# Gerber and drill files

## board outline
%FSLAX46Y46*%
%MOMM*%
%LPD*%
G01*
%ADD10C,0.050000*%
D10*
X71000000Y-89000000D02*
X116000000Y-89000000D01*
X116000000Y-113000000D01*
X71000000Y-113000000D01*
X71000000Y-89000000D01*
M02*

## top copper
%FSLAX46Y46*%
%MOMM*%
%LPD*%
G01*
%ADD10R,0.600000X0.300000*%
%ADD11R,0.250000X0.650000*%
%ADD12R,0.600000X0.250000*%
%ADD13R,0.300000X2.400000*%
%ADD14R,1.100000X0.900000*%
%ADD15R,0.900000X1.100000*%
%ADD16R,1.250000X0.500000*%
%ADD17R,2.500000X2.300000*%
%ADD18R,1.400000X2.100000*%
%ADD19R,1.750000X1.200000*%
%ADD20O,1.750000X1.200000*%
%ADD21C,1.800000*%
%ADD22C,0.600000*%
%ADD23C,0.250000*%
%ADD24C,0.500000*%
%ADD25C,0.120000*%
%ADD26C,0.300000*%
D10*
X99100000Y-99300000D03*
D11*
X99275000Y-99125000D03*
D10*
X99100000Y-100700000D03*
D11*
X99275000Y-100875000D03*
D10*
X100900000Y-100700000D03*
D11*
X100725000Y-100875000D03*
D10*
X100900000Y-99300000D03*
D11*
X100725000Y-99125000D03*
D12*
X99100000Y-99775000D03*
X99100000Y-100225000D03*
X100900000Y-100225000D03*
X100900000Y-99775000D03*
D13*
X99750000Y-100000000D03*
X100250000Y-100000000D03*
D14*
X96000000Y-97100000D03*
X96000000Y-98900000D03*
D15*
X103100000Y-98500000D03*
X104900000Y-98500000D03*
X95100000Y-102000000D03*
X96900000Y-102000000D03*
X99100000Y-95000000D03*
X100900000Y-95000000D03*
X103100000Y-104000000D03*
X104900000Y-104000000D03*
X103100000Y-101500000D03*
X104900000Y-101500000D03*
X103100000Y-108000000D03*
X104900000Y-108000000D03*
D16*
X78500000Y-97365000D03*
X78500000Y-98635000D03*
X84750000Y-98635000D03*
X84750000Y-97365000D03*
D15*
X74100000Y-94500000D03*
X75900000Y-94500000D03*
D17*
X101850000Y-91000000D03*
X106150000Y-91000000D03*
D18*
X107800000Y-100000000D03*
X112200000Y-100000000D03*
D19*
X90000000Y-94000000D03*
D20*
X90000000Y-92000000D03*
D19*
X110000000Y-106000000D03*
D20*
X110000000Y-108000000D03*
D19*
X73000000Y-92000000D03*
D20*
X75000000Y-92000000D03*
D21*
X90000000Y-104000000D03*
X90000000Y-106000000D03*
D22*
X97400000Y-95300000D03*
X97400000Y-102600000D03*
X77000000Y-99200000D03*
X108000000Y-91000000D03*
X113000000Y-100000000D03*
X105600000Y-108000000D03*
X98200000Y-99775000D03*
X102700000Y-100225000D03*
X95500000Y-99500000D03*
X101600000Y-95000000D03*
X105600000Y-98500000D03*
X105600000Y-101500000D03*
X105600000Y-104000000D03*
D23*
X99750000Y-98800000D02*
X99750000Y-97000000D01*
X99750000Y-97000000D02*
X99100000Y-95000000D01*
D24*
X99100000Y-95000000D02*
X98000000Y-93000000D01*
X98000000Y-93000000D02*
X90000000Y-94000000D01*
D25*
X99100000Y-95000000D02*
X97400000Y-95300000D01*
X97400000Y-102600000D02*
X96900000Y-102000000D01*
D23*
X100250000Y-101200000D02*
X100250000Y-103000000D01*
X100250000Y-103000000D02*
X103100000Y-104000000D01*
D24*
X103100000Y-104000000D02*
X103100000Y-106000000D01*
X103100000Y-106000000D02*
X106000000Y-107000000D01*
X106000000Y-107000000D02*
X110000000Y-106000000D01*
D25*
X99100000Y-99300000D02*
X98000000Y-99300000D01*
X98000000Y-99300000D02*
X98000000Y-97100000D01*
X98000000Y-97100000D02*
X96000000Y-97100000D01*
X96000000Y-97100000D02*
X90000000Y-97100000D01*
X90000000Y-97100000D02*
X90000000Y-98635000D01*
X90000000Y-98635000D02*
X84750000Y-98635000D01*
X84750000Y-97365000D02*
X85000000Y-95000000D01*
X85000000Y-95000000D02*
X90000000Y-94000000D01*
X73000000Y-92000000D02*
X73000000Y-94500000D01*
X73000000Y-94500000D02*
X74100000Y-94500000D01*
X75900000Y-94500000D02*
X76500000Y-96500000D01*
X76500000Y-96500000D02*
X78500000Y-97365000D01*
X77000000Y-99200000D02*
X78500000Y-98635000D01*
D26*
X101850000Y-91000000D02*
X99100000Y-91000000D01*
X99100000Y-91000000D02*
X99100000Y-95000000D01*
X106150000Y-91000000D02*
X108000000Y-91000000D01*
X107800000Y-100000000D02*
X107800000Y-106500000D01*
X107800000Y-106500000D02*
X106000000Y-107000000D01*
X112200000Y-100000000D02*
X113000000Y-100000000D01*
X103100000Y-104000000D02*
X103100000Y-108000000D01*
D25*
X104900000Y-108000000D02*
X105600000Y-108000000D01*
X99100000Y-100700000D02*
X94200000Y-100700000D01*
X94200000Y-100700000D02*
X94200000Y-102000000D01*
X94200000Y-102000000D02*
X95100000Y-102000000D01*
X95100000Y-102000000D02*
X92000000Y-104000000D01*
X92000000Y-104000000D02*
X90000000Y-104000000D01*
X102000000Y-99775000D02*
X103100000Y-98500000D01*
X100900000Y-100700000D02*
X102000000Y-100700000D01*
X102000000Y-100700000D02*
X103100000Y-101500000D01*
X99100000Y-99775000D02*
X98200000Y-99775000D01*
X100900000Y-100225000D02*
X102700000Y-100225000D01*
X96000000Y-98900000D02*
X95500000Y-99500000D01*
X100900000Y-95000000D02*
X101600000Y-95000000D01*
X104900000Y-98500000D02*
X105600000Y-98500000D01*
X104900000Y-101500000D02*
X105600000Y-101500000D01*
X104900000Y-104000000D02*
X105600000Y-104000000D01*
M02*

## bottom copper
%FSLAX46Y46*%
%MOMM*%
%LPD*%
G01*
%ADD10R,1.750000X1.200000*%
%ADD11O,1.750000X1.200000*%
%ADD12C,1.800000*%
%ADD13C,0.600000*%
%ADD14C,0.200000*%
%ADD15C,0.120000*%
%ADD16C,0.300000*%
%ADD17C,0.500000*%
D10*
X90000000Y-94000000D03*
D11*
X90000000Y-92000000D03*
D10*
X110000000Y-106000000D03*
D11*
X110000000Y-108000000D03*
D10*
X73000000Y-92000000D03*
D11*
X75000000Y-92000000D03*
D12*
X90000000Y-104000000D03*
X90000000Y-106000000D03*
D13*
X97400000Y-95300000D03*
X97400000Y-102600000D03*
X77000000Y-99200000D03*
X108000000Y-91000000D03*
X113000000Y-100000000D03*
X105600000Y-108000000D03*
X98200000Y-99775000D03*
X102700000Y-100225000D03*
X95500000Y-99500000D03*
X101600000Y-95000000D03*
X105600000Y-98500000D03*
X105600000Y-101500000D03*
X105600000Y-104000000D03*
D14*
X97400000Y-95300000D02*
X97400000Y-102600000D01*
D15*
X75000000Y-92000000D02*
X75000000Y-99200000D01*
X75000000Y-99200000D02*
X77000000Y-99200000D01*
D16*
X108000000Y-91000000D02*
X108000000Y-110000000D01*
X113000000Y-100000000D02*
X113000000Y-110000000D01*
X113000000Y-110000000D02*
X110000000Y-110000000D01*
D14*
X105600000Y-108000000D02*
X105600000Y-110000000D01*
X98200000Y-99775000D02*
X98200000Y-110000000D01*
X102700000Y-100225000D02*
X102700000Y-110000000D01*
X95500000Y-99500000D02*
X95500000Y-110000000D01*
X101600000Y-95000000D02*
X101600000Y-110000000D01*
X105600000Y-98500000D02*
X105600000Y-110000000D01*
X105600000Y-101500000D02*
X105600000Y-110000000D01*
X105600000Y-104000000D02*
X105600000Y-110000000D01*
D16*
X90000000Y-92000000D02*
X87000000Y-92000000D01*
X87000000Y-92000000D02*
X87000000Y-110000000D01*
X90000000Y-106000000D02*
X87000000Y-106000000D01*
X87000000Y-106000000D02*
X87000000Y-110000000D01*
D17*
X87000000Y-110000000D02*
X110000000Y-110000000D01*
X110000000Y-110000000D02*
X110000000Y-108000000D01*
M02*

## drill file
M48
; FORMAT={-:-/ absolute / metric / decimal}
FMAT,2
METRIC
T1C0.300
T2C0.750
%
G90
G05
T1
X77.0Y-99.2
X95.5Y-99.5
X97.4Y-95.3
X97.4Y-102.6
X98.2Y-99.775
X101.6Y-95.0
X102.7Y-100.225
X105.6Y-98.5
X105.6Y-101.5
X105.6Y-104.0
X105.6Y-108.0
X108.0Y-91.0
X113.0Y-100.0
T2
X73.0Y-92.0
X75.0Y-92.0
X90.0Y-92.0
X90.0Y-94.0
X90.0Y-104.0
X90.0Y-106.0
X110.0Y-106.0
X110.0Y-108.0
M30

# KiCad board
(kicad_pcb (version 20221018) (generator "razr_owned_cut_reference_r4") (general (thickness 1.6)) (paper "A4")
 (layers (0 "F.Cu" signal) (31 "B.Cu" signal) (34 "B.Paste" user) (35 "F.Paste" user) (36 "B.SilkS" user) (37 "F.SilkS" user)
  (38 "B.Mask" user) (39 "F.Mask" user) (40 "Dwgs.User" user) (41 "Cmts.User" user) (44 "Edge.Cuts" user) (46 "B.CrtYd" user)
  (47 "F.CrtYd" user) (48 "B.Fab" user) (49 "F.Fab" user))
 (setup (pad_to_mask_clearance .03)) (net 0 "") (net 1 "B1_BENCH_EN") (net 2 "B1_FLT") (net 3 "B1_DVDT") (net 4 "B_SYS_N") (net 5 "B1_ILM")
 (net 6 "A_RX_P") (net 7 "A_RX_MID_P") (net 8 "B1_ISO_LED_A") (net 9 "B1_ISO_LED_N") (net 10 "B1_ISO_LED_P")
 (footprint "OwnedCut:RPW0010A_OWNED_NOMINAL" (layer "F.Cu") (at 100 100)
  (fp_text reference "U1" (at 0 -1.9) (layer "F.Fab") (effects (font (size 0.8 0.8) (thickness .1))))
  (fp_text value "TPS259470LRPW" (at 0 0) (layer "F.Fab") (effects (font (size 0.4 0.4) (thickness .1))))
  (pad "1" smd rect (at -0.9 -0.7) (size 0.6 0.3) (layers "F.Cu" "F.Paste" "F.Mask") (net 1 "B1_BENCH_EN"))
  (pad "1" smd rect (at -0.725 -0.875) (size 0.25 0.65) (layers "F.Cu" "F.Paste" "F.Mask") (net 1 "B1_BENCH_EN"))
  (pad "4" smd rect (at -0.9 0.7) (size 0.6 0.3) (layers "F.Cu" "F.Paste" "F.Mask") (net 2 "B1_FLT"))
  (pad "4" smd rect (at -0.725 0.875) (size 0.25 0.65) (layers "F.Cu" "F.Paste" "F.Mask") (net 2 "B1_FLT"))
  (pad "7" smd rect (at 0.9 0.7) (size 0.6 0.3) (layers "F.Cu" "F.Paste" "F.Mask") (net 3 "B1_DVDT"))
  (pad "7" smd rect (at 0.725 0.875) (size 0.25 0.65) (layers "F.Cu" "F.Paste" "F.Mask") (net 3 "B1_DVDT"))
  (pad "10" smd rect (at 0.9 -0.7) (size 0.6 0.3) (layers "F.Cu" "F.Paste" "F.Mask"))
  (pad "10" smd rect (at 0.725 -0.875) (size 0.25 0.65) (layers "F.Cu" "F.Paste" "F.Mask"))
  (pad "2" smd rect (at -0.9 -0.225) (size 0.6 0.25) (layers "F.Cu" "F.Paste" "F.Mask") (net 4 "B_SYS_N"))
  (pad "3" smd rect (at -0.9 0.225) (size 0.6 0.25) (layers "F.Cu" "F.Paste" "F.Mask"))
  (pad "8" smd rect (at 0.9 0.225) (size 0.6 0.25) (layers "F.Cu" "F.Paste" "F.Mask") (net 4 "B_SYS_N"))
  (pad "9" smd rect (at 0.9 -0.225) (size 0.6 0.25) (layers "F.Cu" "F.Paste" "F.Mask") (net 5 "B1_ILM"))
  (pad "5" smd rect (at -0.25 0) (size 0.3 2.4) (layers "F.Cu" "F.Paste" "F.Mask") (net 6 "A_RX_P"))
  (pad "6" smd rect (at 0.25 0) (size 0.3 2.4) (layers "F.Cu" "F.Paste" "F.Mask") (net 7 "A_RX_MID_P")))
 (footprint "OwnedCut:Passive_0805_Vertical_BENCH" (layer "F.Cu") (at 96 98)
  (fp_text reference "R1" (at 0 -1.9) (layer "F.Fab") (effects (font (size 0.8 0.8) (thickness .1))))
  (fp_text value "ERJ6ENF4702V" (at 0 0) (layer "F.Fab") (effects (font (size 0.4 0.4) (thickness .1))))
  (pad "1" smd rect (at 0 -0.9) (size 1.1 0.9) (layers "F.Cu" "F.Paste" "F.Mask") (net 1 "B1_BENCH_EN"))
  (pad "2" smd rect (at 0 0.9) (size 1.1 0.9) (layers "F.Cu" "F.Paste" "F.Mask") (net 4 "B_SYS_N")))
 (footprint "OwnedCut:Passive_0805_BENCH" (layer "F.Cu") (at 104 98.5)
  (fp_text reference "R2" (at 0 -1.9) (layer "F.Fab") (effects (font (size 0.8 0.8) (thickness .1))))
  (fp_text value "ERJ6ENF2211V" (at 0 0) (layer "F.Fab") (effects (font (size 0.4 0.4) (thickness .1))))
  (pad "1" smd rect (at -0.9 0) (size 0.9 1.1) (layers "F.Cu" "F.Paste" "F.Mask") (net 5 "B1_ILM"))
  (pad "2" smd rect (at 0.9 0) (size 0.9 1.1) (layers "F.Cu" "F.Paste" "F.Mask") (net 4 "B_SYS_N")))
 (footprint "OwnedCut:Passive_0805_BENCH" (layer "F.Cu") (at 96 102)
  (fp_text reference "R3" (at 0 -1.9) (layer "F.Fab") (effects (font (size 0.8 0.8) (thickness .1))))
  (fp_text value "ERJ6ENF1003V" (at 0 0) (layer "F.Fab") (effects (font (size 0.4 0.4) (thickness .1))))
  (pad "1" smd rect (at -0.9 0) (size 0.9 1.1) (layers "F.Cu" "F.Paste" "F.Mask") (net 2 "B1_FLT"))
  (pad "2" smd rect (at 0.9 0) (size 0.9 1.1) (layers "F.Cu" "F.Paste" "F.Mask") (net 6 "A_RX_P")))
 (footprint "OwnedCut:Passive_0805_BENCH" (layer "F.Cu") (at 100 95)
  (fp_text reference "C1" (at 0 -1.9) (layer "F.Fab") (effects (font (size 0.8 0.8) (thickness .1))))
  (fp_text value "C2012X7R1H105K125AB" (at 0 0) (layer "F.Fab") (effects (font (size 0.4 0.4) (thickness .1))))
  (pad "1" smd rect (at -0.9 0) (size 0.9 1.1) (layers "F.Cu" "F.Paste" "F.Mask") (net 6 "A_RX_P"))
  (pad "2" smd rect (at 0.9 0) (size 0.9 1.1) (layers "F.Cu" "F.Paste" "F.Mask") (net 4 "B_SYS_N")))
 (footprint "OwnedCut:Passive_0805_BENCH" (layer "F.Cu") (at 104 104)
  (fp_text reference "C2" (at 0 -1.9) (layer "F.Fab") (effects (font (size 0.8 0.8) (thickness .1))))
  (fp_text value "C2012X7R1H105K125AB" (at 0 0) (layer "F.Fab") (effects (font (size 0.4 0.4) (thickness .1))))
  (pad "1" smd rect (at -0.9 0) (size 0.9 1.1) (layers "F.Cu" "F.Paste" "F.Mask") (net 7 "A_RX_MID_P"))
  (pad "2" smd rect (at 0.9 0) (size 0.9 1.1) (layers "F.Cu" "F.Paste" "F.Mask") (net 4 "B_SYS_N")))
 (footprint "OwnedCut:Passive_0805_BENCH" (layer "F.Cu") (at 104 101.5)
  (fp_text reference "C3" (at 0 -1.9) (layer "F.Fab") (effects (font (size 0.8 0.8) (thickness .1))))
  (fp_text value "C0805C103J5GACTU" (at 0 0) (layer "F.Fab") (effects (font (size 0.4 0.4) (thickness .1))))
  (pad "1" smd rect (at -0.9 0) (size 0.9 1.1) (layers "F.Cu" "F.Paste" "F.Mask") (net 3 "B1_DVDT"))
  (pad "2" smd rect (at 0.9 0) (size 0.9 1.1) (layers "F.Cu" "F.Paste" "F.Mask") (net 4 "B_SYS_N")))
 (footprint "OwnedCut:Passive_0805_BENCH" (layer "F.Cu") (at 104 108)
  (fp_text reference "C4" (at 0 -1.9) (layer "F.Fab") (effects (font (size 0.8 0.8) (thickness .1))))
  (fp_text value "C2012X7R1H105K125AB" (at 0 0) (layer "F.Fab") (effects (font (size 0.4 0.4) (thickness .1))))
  (pad "1" smd rect (at -0.9 0) (size 0.9 1.1) (layers "F.Cu" "F.Paste" "F.Mask") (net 7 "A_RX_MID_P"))
  (pad "2" smd rect (at 0.9 0) (size 0.9 1.1) (layers "F.Cu" "F.Paste" "F.Mask") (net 4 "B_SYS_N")))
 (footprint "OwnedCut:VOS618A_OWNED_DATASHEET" (layer "F.Cu") (at 81.625 98)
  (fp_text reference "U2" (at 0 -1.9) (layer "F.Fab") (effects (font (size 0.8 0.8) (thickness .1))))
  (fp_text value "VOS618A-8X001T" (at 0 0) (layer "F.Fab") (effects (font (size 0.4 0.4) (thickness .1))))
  (pad "1" smd rect (at -3.125 -0.635) (size 1.25 0.5) (layers "F.Cu" "F.Paste" "F.Mask") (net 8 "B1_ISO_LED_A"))
  (pad "2" smd rect (at -3.125 0.635) (size 1.25 0.5) (layers "F.Cu" "F.Paste" "F.Mask") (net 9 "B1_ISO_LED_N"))
  (pad "3" smd rect (at 3.125 0.635) (size 1.25 0.5) (layers "F.Cu" "F.Paste" "F.Mask") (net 1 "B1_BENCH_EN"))
  (pad "4" smd rect (at 3.125 -0.635) (size 1.25 0.5) (layers "F.Cu" "F.Paste" "F.Mask") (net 6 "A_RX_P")))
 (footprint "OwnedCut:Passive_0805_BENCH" (layer "F.Cu") (at 75 94.5)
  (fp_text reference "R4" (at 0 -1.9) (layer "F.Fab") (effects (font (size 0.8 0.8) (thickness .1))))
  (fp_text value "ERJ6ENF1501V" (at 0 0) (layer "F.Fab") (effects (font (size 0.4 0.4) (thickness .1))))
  (pad "1" smd rect (at -0.9 0) (size 0.9 1.1) (layers "F.Cu" "F.Paste" "F.Mask") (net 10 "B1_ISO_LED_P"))
  (pad "2" smd rect (at 0.9 0) (size 0.9 1.1) (layers "F.Cu" "F.Paste" "F.Mask") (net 8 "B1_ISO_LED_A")))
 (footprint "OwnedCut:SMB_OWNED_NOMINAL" (layer "F.Cu") (at 104 91)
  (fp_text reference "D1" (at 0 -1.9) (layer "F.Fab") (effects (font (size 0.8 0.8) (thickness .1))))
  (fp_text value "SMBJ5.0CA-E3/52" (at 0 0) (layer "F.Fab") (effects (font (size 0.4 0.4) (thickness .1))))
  (pad "1" smd rect (at -2.15 0) (size 2.5 2.3) (layers "F.Cu" "F.Paste" "F.Mask") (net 6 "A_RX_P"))
  (pad "2" smd rect (at 2.15 0) (size 2.5 2.3) (layers "F.Cu" "F.Paste" "F.Mask") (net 4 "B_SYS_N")))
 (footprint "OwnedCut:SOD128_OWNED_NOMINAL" (layer "F.Cu") (at 110 100)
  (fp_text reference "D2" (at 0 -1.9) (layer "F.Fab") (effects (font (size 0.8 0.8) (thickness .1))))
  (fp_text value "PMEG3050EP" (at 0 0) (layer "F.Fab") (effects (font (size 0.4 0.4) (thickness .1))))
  (pad "1" smd rect (at -2.2 0) (size 1.4 2.1) (layers "F.Cu" "F.Paste" "F.Mask") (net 7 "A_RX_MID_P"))
  (pad "2" smd rect (at 2.2 0) (size 1.4 2.1) (layers "F.Cu" "F.Paste" "F.Mask") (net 4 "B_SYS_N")))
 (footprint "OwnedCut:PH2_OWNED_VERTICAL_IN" (layer "F.Cu") (at 90 94)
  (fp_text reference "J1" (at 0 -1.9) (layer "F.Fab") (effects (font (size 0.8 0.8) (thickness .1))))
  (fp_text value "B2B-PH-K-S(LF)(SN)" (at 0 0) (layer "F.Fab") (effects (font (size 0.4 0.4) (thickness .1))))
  (pad "1" thru_hole rect (at 0 0) (size 1.75 1.2) (drill .75) (layers "*.Cu" "*.Mask") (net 6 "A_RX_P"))
  (pad "2" thru_hole oval (at 0 -2) (size 1.75 1.2) (drill .75) (layers "*.Cu" "*.Mask") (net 4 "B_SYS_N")))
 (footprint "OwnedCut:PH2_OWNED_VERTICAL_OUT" (layer "F.Cu") (at 110 106)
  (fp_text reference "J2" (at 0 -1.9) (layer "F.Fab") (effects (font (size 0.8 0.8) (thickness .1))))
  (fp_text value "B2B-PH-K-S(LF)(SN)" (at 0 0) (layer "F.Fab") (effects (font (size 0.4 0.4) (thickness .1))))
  (pad "1" thru_hole rect (at 0 0) (size 1.75 1.2) (drill .75) (layers "*.Cu" "*.Mask") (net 7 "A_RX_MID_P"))
  (pad "2" thru_hole oval (at 0 2) (size 1.75 1.2) (drill .75) (layers "*.Cu" "*.Mask") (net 4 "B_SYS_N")))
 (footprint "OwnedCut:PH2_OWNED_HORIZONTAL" (layer "F.Cu") (at 73 92)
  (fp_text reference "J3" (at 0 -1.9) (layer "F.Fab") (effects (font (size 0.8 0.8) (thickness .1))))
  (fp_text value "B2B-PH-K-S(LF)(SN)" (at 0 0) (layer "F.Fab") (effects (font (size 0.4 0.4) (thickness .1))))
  (pad "1" thru_hole rect (at 0 0) (size 1.75 1.2) (drill .75) (layers "*.Cu" "*.Mask") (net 10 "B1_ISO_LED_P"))
  (pad "2" thru_hole oval (at 2 0) (size 1.75 1.2) (drill .75) (layers "*.Cu" "*.Mask") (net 9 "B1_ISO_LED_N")))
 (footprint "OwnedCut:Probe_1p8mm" (layer "F.Cu") (at 90 104)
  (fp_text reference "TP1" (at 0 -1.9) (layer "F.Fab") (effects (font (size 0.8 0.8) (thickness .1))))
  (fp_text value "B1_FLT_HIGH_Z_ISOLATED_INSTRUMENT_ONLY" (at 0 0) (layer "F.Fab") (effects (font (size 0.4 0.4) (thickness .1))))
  (pad "1" thru_hole circle (at 0 0) (size 1.8 1.8) (drill .75) (layers "*.Cu" "*.Mask") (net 2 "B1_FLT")))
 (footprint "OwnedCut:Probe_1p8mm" (layer "F.Cu") (at 90 106)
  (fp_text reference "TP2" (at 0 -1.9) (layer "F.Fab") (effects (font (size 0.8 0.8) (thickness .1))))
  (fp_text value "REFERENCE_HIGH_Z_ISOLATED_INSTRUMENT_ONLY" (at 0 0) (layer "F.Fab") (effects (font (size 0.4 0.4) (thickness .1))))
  (pad "1" thru_hole circle (at 0 0) (size 1.8 1.8) (drill .75) (layers "*.Cu" "*.Mask") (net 4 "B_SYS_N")))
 (segment (start 99.75 98.8) (end 99.75 97) (width 0.25) (layer "F.Cu") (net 6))
 (segment (start 99.75 97) (end 99.1 95) (width 0.25) (layer "F.Cu") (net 6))
 (segment (start 99.1 95) (end 98 93) (width 0.5) (layer "F.Cu") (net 6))
 (segment (start 98 93) (end 90 94) (width 0.5) (layer "F.Cu") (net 6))
 (segment (start 99.1 95) (end 97.4 95.3) (width 0.12) (layer "F.Cu") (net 6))
 (via (at 97.4 95.3) (size .6) (drill .3) (layers "F.Cu" "B.Cu") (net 6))
 (segment (start 97.4 95.3) (end 97.4 102.6) (width 0.2) (layer "B.Cu") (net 6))
 (via (at 97.4 102.6) (size .6) (drill .3) (layers "F.Cu" "B.Cu") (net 6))
 (segment (start 97.4 102.6) (end 96.9 102) (width 0.12) (layer "F.Cu") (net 6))
 (segment (start 100.25 101.2) (end 100.25 103) (width 0.25) (layer "F.Cu") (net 7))
 (segment (start 100.25 103) (end 103.1 104) (width 0.25) (layer "F.Cu") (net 7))
 (segment (start 103.1 104) (end 103.1 106) (width 0.5) (layer "F.Cu") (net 7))
 (segment (start 103.1 106) (end 106 107) (width 0.5) (layer "F.Cu") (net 7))
 (segment (start 106 107) (end 110 106) (width 0.5) (layer "F.Cu") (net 7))
 (segment (start 99.1 99.3) (end 98 99.3) (width 0.12) (layer "F.Cu") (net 1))
 (segment (start 98 99.3) (end 98 97.1) (width 0.12) (layer "F.Cu") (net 1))
 (segment (start 98 97.1) (end 96 97.1) (width 0.12) (layer "F.Cu") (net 1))
 (segment (start 96 97.1) (end 90 97.1) (width 0.12) (layer "F.Cu") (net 1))
 (segment (start 90 97.1) (end 90 98.635) (width 0.12) (layer "F.Cu") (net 1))
 (segment (start 90 98.635) (end 84.75 98.635) (width 0.12) (layer "F.Cu") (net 1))
 (segment (start 84.75 97.365) (end 85 95) (width 0.12) (layer "F.Cu") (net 6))
 (segment (start 85 95) (end 90 94) (width 0.12) (layer "F.Cu") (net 6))
 (segment (start 73 92) (end 73 94.5) (width 0.12) (layer "F.Cu") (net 10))
 (segment (start 73 94.5) (end 74.1 94.5) (width 0.12) (layer "F.Cu") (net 10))
 (segment (start 75.9 94.5) (end 76.5 96.5) (width 0.12) (layer "F.Cu") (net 8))
 (segment (start 76.5 96.5) (end 78.5 97.365) (width 0.12) (layer "F.Cu") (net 8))
 (segment (start 75 92) (end 75 99.2) (width 0.12) (layer "B.Cu") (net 9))
 (segment (start 75 99.2) (end 77 99.2) (width 0.12) (layer "B.Cu") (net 9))
 (via (at 77 99.2) (size .6) (drill .3) (layers "F.Cu" "B.Cu") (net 9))
 (segment (start 77 99.2) (end 78.5 98.635) (width 0.12) (layer "F.Cu") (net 9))
 (segment (start 101.85 91) (end 99.1 91) (width 0.3) (layer "F.Cu") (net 6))
 (segment (start 99.1 91) (end 99.1 95) (width 0.3) (layer "F.Cu") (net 6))
 (segment (start 106.15 91) (end 108 91) (width 0.3) (layer "F.Cu") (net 4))
 (via (at 108 91) (size .6) (drill .3) (layers "F.Cu" "B.Cu") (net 4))
 (segment (start 108 91) (end 108 110) (width 0.3) (layer "B.Cu") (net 4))
 (segment (start 107.8 100) (end 107.8 106.5) (width 0.3) (layer "F.Cu") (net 7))
 (segment (start 107.8 106.5) (end 106 107) (width 0.3) (layer "F.Cu") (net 7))
 (segment (start 112.2 100) (end 113 100) (width 0.3) (layer "F.Cu") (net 4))
 (via (at 113 100) (size .6) (drill .3) (layers "F.Cu" "B.Cu") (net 4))
 (segment (start 113 100) (end 113 110) (width 0.3) (layer "B.Cu") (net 4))
 (segment (start 113 110) (end 110 110) (width 0.3) (layer "B.Cu") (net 4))
 (segment (start 103.1 104) (end 103.1 108) (width 0.3) (layer "F.Cu") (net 7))
 (segment (start 104.9 108) (end 105.6 108) (width 0.12) (layer "F.Cu") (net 4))
 (via (at 105.6 108) (size .6) (drill .3) (layers "F.Cu" "B.Cu") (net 4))
 (segment (start 105.6 108) (end 105.6 110) (width 0.2) (layer "B.Cu") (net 4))
 (segment (start 99.1 100.7) (end 94.2 100.7) (width 0.12) (layer "F.Cu") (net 2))
 (segment (start 94.2 100.7) (end 94.2 102) (width 0.12) (layer "F.Cu") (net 2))
 (segment (start 94.2 102) (end 95.1 102) (width 0.12) (layer "F.Cu") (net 2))
 (segment (start 95.1 102) (end 92 104) (width 0.12) (layer "F.Cu") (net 2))
 (segment (start 92 104) (end 90 104) (width 0.12) (layer "F.Cu") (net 2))
 (segment (start 102 99.775) (end 103.1 98.5) (width 0.12) (layer "F.Cu") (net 5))
 (segment (start 100.9 100.7) (end 102 100.7) (width 0.12) (layer "F.Cu") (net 3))
 (segment (start 102 100.7) (end 103.1 101.5) (width 0.12) (layer "F.Cu") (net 3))
 (segment (start 99.1 99.775) (end 98.2 99.775) (width 0.12) (layer "F.Cu") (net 4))
 (via (at 98.2 99.775) (size .6) (drill .3) (layers "F.Cu" "B.Cu") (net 4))
 (segment (start 98.2 99.775) (end 98.2 110) (width 0.2) (layer "B.Cu") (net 4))
 (segment (start 100.9 100.225) (end 102.7 100.225) (width 0.12) (layer "F.Cu") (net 4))
 (via (at 102.7 100.225) (size .6) (drill .3) (layers "F.Cu" "B.Cu") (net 4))
 (segment (start 102.7 100.225) (end 102.7 110) (width 0.2) (layer "B.Cu") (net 4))
 (segment (start 96 98.9) (end 95.5 99.5) (width 0.12) (layer "F.Cu") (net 4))
 (via (at 95.5 99.5) (size .6) (drill .3) (layers "F.Cu" "B.Cu") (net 4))
 (segment (start 95.5 99.5) (end 95.5 110) (width 0.2) (layer "B.Cu") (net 4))
 (segment (start 100.9 95) (end 101.6 95) (width 0.12) (layer "F.Cu") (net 4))
 (via (at 101.6 95) (size .6) (drill .3) (layers "F.Cu" "B.Cu") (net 4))
 (segment (start 101.6 95) (end 101.6 110) (width 0.2) (layer "B.Cu") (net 4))
 (segment (start 104.9 98.5) (end 105.6 98.5) (width 0.12) (layer "F.Cu") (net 4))
 (via (at 105.6 98.5) (size .6) (drill .3) (layers "F.Cu" "B.Cu") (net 4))
 (segment (start 105.6 98.5) (end 105.6 110) (width 0.2) (layer "B.Cu") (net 4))
 (segment (start 104.9 101.5) (end 105.6 101.5) (width 0.12) (layer "F.Cu") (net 4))
 (via (at 105.6 101.5) (size .6) (drill .3) (layers "F.Cu" "B.Cu") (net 4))
 (segment (start 105.6 101.5) (end 105.6 110) (width 0.2) (layer "B.Cu") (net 4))
 (segment (start 104.9 104) (end 105.6 104) (width 0.12) (layer "F.Cu") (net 4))
 (via (at 105.6 104) (size .6) (drill .3) (layers "F.Cu" "B.Cu") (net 4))
 (segment (start 105.6 104) (end 105.6 110) (width 0.2) (layer "B.Cu") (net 4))
 (segment (start 90 92) (end 87 92) (width 0.3) (layer "B.Cu") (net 4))
 (segment (start 87 92) (end 87 110) (width 0.3) (layer "B.Cu") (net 4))
 (segment (start 90 106) (end 87 106) (width 0.3) (layer "B.Cu") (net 4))
 (segment (start 87 106) (end 87 110) (width 0.3) (layer "B.Cu") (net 4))
 (segment (start 87 110) (end 110 110) (width 0.5) (layer "B.Cu") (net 4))
 (segment (start 110 110) (end 110 108) (width 0.5) (layer "B.Cu") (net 4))
 (gr_rect (start 71 89) (end 116 113) (stroke (width .05) (type default)) (fill none) (layer "Edge.Cuts")))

